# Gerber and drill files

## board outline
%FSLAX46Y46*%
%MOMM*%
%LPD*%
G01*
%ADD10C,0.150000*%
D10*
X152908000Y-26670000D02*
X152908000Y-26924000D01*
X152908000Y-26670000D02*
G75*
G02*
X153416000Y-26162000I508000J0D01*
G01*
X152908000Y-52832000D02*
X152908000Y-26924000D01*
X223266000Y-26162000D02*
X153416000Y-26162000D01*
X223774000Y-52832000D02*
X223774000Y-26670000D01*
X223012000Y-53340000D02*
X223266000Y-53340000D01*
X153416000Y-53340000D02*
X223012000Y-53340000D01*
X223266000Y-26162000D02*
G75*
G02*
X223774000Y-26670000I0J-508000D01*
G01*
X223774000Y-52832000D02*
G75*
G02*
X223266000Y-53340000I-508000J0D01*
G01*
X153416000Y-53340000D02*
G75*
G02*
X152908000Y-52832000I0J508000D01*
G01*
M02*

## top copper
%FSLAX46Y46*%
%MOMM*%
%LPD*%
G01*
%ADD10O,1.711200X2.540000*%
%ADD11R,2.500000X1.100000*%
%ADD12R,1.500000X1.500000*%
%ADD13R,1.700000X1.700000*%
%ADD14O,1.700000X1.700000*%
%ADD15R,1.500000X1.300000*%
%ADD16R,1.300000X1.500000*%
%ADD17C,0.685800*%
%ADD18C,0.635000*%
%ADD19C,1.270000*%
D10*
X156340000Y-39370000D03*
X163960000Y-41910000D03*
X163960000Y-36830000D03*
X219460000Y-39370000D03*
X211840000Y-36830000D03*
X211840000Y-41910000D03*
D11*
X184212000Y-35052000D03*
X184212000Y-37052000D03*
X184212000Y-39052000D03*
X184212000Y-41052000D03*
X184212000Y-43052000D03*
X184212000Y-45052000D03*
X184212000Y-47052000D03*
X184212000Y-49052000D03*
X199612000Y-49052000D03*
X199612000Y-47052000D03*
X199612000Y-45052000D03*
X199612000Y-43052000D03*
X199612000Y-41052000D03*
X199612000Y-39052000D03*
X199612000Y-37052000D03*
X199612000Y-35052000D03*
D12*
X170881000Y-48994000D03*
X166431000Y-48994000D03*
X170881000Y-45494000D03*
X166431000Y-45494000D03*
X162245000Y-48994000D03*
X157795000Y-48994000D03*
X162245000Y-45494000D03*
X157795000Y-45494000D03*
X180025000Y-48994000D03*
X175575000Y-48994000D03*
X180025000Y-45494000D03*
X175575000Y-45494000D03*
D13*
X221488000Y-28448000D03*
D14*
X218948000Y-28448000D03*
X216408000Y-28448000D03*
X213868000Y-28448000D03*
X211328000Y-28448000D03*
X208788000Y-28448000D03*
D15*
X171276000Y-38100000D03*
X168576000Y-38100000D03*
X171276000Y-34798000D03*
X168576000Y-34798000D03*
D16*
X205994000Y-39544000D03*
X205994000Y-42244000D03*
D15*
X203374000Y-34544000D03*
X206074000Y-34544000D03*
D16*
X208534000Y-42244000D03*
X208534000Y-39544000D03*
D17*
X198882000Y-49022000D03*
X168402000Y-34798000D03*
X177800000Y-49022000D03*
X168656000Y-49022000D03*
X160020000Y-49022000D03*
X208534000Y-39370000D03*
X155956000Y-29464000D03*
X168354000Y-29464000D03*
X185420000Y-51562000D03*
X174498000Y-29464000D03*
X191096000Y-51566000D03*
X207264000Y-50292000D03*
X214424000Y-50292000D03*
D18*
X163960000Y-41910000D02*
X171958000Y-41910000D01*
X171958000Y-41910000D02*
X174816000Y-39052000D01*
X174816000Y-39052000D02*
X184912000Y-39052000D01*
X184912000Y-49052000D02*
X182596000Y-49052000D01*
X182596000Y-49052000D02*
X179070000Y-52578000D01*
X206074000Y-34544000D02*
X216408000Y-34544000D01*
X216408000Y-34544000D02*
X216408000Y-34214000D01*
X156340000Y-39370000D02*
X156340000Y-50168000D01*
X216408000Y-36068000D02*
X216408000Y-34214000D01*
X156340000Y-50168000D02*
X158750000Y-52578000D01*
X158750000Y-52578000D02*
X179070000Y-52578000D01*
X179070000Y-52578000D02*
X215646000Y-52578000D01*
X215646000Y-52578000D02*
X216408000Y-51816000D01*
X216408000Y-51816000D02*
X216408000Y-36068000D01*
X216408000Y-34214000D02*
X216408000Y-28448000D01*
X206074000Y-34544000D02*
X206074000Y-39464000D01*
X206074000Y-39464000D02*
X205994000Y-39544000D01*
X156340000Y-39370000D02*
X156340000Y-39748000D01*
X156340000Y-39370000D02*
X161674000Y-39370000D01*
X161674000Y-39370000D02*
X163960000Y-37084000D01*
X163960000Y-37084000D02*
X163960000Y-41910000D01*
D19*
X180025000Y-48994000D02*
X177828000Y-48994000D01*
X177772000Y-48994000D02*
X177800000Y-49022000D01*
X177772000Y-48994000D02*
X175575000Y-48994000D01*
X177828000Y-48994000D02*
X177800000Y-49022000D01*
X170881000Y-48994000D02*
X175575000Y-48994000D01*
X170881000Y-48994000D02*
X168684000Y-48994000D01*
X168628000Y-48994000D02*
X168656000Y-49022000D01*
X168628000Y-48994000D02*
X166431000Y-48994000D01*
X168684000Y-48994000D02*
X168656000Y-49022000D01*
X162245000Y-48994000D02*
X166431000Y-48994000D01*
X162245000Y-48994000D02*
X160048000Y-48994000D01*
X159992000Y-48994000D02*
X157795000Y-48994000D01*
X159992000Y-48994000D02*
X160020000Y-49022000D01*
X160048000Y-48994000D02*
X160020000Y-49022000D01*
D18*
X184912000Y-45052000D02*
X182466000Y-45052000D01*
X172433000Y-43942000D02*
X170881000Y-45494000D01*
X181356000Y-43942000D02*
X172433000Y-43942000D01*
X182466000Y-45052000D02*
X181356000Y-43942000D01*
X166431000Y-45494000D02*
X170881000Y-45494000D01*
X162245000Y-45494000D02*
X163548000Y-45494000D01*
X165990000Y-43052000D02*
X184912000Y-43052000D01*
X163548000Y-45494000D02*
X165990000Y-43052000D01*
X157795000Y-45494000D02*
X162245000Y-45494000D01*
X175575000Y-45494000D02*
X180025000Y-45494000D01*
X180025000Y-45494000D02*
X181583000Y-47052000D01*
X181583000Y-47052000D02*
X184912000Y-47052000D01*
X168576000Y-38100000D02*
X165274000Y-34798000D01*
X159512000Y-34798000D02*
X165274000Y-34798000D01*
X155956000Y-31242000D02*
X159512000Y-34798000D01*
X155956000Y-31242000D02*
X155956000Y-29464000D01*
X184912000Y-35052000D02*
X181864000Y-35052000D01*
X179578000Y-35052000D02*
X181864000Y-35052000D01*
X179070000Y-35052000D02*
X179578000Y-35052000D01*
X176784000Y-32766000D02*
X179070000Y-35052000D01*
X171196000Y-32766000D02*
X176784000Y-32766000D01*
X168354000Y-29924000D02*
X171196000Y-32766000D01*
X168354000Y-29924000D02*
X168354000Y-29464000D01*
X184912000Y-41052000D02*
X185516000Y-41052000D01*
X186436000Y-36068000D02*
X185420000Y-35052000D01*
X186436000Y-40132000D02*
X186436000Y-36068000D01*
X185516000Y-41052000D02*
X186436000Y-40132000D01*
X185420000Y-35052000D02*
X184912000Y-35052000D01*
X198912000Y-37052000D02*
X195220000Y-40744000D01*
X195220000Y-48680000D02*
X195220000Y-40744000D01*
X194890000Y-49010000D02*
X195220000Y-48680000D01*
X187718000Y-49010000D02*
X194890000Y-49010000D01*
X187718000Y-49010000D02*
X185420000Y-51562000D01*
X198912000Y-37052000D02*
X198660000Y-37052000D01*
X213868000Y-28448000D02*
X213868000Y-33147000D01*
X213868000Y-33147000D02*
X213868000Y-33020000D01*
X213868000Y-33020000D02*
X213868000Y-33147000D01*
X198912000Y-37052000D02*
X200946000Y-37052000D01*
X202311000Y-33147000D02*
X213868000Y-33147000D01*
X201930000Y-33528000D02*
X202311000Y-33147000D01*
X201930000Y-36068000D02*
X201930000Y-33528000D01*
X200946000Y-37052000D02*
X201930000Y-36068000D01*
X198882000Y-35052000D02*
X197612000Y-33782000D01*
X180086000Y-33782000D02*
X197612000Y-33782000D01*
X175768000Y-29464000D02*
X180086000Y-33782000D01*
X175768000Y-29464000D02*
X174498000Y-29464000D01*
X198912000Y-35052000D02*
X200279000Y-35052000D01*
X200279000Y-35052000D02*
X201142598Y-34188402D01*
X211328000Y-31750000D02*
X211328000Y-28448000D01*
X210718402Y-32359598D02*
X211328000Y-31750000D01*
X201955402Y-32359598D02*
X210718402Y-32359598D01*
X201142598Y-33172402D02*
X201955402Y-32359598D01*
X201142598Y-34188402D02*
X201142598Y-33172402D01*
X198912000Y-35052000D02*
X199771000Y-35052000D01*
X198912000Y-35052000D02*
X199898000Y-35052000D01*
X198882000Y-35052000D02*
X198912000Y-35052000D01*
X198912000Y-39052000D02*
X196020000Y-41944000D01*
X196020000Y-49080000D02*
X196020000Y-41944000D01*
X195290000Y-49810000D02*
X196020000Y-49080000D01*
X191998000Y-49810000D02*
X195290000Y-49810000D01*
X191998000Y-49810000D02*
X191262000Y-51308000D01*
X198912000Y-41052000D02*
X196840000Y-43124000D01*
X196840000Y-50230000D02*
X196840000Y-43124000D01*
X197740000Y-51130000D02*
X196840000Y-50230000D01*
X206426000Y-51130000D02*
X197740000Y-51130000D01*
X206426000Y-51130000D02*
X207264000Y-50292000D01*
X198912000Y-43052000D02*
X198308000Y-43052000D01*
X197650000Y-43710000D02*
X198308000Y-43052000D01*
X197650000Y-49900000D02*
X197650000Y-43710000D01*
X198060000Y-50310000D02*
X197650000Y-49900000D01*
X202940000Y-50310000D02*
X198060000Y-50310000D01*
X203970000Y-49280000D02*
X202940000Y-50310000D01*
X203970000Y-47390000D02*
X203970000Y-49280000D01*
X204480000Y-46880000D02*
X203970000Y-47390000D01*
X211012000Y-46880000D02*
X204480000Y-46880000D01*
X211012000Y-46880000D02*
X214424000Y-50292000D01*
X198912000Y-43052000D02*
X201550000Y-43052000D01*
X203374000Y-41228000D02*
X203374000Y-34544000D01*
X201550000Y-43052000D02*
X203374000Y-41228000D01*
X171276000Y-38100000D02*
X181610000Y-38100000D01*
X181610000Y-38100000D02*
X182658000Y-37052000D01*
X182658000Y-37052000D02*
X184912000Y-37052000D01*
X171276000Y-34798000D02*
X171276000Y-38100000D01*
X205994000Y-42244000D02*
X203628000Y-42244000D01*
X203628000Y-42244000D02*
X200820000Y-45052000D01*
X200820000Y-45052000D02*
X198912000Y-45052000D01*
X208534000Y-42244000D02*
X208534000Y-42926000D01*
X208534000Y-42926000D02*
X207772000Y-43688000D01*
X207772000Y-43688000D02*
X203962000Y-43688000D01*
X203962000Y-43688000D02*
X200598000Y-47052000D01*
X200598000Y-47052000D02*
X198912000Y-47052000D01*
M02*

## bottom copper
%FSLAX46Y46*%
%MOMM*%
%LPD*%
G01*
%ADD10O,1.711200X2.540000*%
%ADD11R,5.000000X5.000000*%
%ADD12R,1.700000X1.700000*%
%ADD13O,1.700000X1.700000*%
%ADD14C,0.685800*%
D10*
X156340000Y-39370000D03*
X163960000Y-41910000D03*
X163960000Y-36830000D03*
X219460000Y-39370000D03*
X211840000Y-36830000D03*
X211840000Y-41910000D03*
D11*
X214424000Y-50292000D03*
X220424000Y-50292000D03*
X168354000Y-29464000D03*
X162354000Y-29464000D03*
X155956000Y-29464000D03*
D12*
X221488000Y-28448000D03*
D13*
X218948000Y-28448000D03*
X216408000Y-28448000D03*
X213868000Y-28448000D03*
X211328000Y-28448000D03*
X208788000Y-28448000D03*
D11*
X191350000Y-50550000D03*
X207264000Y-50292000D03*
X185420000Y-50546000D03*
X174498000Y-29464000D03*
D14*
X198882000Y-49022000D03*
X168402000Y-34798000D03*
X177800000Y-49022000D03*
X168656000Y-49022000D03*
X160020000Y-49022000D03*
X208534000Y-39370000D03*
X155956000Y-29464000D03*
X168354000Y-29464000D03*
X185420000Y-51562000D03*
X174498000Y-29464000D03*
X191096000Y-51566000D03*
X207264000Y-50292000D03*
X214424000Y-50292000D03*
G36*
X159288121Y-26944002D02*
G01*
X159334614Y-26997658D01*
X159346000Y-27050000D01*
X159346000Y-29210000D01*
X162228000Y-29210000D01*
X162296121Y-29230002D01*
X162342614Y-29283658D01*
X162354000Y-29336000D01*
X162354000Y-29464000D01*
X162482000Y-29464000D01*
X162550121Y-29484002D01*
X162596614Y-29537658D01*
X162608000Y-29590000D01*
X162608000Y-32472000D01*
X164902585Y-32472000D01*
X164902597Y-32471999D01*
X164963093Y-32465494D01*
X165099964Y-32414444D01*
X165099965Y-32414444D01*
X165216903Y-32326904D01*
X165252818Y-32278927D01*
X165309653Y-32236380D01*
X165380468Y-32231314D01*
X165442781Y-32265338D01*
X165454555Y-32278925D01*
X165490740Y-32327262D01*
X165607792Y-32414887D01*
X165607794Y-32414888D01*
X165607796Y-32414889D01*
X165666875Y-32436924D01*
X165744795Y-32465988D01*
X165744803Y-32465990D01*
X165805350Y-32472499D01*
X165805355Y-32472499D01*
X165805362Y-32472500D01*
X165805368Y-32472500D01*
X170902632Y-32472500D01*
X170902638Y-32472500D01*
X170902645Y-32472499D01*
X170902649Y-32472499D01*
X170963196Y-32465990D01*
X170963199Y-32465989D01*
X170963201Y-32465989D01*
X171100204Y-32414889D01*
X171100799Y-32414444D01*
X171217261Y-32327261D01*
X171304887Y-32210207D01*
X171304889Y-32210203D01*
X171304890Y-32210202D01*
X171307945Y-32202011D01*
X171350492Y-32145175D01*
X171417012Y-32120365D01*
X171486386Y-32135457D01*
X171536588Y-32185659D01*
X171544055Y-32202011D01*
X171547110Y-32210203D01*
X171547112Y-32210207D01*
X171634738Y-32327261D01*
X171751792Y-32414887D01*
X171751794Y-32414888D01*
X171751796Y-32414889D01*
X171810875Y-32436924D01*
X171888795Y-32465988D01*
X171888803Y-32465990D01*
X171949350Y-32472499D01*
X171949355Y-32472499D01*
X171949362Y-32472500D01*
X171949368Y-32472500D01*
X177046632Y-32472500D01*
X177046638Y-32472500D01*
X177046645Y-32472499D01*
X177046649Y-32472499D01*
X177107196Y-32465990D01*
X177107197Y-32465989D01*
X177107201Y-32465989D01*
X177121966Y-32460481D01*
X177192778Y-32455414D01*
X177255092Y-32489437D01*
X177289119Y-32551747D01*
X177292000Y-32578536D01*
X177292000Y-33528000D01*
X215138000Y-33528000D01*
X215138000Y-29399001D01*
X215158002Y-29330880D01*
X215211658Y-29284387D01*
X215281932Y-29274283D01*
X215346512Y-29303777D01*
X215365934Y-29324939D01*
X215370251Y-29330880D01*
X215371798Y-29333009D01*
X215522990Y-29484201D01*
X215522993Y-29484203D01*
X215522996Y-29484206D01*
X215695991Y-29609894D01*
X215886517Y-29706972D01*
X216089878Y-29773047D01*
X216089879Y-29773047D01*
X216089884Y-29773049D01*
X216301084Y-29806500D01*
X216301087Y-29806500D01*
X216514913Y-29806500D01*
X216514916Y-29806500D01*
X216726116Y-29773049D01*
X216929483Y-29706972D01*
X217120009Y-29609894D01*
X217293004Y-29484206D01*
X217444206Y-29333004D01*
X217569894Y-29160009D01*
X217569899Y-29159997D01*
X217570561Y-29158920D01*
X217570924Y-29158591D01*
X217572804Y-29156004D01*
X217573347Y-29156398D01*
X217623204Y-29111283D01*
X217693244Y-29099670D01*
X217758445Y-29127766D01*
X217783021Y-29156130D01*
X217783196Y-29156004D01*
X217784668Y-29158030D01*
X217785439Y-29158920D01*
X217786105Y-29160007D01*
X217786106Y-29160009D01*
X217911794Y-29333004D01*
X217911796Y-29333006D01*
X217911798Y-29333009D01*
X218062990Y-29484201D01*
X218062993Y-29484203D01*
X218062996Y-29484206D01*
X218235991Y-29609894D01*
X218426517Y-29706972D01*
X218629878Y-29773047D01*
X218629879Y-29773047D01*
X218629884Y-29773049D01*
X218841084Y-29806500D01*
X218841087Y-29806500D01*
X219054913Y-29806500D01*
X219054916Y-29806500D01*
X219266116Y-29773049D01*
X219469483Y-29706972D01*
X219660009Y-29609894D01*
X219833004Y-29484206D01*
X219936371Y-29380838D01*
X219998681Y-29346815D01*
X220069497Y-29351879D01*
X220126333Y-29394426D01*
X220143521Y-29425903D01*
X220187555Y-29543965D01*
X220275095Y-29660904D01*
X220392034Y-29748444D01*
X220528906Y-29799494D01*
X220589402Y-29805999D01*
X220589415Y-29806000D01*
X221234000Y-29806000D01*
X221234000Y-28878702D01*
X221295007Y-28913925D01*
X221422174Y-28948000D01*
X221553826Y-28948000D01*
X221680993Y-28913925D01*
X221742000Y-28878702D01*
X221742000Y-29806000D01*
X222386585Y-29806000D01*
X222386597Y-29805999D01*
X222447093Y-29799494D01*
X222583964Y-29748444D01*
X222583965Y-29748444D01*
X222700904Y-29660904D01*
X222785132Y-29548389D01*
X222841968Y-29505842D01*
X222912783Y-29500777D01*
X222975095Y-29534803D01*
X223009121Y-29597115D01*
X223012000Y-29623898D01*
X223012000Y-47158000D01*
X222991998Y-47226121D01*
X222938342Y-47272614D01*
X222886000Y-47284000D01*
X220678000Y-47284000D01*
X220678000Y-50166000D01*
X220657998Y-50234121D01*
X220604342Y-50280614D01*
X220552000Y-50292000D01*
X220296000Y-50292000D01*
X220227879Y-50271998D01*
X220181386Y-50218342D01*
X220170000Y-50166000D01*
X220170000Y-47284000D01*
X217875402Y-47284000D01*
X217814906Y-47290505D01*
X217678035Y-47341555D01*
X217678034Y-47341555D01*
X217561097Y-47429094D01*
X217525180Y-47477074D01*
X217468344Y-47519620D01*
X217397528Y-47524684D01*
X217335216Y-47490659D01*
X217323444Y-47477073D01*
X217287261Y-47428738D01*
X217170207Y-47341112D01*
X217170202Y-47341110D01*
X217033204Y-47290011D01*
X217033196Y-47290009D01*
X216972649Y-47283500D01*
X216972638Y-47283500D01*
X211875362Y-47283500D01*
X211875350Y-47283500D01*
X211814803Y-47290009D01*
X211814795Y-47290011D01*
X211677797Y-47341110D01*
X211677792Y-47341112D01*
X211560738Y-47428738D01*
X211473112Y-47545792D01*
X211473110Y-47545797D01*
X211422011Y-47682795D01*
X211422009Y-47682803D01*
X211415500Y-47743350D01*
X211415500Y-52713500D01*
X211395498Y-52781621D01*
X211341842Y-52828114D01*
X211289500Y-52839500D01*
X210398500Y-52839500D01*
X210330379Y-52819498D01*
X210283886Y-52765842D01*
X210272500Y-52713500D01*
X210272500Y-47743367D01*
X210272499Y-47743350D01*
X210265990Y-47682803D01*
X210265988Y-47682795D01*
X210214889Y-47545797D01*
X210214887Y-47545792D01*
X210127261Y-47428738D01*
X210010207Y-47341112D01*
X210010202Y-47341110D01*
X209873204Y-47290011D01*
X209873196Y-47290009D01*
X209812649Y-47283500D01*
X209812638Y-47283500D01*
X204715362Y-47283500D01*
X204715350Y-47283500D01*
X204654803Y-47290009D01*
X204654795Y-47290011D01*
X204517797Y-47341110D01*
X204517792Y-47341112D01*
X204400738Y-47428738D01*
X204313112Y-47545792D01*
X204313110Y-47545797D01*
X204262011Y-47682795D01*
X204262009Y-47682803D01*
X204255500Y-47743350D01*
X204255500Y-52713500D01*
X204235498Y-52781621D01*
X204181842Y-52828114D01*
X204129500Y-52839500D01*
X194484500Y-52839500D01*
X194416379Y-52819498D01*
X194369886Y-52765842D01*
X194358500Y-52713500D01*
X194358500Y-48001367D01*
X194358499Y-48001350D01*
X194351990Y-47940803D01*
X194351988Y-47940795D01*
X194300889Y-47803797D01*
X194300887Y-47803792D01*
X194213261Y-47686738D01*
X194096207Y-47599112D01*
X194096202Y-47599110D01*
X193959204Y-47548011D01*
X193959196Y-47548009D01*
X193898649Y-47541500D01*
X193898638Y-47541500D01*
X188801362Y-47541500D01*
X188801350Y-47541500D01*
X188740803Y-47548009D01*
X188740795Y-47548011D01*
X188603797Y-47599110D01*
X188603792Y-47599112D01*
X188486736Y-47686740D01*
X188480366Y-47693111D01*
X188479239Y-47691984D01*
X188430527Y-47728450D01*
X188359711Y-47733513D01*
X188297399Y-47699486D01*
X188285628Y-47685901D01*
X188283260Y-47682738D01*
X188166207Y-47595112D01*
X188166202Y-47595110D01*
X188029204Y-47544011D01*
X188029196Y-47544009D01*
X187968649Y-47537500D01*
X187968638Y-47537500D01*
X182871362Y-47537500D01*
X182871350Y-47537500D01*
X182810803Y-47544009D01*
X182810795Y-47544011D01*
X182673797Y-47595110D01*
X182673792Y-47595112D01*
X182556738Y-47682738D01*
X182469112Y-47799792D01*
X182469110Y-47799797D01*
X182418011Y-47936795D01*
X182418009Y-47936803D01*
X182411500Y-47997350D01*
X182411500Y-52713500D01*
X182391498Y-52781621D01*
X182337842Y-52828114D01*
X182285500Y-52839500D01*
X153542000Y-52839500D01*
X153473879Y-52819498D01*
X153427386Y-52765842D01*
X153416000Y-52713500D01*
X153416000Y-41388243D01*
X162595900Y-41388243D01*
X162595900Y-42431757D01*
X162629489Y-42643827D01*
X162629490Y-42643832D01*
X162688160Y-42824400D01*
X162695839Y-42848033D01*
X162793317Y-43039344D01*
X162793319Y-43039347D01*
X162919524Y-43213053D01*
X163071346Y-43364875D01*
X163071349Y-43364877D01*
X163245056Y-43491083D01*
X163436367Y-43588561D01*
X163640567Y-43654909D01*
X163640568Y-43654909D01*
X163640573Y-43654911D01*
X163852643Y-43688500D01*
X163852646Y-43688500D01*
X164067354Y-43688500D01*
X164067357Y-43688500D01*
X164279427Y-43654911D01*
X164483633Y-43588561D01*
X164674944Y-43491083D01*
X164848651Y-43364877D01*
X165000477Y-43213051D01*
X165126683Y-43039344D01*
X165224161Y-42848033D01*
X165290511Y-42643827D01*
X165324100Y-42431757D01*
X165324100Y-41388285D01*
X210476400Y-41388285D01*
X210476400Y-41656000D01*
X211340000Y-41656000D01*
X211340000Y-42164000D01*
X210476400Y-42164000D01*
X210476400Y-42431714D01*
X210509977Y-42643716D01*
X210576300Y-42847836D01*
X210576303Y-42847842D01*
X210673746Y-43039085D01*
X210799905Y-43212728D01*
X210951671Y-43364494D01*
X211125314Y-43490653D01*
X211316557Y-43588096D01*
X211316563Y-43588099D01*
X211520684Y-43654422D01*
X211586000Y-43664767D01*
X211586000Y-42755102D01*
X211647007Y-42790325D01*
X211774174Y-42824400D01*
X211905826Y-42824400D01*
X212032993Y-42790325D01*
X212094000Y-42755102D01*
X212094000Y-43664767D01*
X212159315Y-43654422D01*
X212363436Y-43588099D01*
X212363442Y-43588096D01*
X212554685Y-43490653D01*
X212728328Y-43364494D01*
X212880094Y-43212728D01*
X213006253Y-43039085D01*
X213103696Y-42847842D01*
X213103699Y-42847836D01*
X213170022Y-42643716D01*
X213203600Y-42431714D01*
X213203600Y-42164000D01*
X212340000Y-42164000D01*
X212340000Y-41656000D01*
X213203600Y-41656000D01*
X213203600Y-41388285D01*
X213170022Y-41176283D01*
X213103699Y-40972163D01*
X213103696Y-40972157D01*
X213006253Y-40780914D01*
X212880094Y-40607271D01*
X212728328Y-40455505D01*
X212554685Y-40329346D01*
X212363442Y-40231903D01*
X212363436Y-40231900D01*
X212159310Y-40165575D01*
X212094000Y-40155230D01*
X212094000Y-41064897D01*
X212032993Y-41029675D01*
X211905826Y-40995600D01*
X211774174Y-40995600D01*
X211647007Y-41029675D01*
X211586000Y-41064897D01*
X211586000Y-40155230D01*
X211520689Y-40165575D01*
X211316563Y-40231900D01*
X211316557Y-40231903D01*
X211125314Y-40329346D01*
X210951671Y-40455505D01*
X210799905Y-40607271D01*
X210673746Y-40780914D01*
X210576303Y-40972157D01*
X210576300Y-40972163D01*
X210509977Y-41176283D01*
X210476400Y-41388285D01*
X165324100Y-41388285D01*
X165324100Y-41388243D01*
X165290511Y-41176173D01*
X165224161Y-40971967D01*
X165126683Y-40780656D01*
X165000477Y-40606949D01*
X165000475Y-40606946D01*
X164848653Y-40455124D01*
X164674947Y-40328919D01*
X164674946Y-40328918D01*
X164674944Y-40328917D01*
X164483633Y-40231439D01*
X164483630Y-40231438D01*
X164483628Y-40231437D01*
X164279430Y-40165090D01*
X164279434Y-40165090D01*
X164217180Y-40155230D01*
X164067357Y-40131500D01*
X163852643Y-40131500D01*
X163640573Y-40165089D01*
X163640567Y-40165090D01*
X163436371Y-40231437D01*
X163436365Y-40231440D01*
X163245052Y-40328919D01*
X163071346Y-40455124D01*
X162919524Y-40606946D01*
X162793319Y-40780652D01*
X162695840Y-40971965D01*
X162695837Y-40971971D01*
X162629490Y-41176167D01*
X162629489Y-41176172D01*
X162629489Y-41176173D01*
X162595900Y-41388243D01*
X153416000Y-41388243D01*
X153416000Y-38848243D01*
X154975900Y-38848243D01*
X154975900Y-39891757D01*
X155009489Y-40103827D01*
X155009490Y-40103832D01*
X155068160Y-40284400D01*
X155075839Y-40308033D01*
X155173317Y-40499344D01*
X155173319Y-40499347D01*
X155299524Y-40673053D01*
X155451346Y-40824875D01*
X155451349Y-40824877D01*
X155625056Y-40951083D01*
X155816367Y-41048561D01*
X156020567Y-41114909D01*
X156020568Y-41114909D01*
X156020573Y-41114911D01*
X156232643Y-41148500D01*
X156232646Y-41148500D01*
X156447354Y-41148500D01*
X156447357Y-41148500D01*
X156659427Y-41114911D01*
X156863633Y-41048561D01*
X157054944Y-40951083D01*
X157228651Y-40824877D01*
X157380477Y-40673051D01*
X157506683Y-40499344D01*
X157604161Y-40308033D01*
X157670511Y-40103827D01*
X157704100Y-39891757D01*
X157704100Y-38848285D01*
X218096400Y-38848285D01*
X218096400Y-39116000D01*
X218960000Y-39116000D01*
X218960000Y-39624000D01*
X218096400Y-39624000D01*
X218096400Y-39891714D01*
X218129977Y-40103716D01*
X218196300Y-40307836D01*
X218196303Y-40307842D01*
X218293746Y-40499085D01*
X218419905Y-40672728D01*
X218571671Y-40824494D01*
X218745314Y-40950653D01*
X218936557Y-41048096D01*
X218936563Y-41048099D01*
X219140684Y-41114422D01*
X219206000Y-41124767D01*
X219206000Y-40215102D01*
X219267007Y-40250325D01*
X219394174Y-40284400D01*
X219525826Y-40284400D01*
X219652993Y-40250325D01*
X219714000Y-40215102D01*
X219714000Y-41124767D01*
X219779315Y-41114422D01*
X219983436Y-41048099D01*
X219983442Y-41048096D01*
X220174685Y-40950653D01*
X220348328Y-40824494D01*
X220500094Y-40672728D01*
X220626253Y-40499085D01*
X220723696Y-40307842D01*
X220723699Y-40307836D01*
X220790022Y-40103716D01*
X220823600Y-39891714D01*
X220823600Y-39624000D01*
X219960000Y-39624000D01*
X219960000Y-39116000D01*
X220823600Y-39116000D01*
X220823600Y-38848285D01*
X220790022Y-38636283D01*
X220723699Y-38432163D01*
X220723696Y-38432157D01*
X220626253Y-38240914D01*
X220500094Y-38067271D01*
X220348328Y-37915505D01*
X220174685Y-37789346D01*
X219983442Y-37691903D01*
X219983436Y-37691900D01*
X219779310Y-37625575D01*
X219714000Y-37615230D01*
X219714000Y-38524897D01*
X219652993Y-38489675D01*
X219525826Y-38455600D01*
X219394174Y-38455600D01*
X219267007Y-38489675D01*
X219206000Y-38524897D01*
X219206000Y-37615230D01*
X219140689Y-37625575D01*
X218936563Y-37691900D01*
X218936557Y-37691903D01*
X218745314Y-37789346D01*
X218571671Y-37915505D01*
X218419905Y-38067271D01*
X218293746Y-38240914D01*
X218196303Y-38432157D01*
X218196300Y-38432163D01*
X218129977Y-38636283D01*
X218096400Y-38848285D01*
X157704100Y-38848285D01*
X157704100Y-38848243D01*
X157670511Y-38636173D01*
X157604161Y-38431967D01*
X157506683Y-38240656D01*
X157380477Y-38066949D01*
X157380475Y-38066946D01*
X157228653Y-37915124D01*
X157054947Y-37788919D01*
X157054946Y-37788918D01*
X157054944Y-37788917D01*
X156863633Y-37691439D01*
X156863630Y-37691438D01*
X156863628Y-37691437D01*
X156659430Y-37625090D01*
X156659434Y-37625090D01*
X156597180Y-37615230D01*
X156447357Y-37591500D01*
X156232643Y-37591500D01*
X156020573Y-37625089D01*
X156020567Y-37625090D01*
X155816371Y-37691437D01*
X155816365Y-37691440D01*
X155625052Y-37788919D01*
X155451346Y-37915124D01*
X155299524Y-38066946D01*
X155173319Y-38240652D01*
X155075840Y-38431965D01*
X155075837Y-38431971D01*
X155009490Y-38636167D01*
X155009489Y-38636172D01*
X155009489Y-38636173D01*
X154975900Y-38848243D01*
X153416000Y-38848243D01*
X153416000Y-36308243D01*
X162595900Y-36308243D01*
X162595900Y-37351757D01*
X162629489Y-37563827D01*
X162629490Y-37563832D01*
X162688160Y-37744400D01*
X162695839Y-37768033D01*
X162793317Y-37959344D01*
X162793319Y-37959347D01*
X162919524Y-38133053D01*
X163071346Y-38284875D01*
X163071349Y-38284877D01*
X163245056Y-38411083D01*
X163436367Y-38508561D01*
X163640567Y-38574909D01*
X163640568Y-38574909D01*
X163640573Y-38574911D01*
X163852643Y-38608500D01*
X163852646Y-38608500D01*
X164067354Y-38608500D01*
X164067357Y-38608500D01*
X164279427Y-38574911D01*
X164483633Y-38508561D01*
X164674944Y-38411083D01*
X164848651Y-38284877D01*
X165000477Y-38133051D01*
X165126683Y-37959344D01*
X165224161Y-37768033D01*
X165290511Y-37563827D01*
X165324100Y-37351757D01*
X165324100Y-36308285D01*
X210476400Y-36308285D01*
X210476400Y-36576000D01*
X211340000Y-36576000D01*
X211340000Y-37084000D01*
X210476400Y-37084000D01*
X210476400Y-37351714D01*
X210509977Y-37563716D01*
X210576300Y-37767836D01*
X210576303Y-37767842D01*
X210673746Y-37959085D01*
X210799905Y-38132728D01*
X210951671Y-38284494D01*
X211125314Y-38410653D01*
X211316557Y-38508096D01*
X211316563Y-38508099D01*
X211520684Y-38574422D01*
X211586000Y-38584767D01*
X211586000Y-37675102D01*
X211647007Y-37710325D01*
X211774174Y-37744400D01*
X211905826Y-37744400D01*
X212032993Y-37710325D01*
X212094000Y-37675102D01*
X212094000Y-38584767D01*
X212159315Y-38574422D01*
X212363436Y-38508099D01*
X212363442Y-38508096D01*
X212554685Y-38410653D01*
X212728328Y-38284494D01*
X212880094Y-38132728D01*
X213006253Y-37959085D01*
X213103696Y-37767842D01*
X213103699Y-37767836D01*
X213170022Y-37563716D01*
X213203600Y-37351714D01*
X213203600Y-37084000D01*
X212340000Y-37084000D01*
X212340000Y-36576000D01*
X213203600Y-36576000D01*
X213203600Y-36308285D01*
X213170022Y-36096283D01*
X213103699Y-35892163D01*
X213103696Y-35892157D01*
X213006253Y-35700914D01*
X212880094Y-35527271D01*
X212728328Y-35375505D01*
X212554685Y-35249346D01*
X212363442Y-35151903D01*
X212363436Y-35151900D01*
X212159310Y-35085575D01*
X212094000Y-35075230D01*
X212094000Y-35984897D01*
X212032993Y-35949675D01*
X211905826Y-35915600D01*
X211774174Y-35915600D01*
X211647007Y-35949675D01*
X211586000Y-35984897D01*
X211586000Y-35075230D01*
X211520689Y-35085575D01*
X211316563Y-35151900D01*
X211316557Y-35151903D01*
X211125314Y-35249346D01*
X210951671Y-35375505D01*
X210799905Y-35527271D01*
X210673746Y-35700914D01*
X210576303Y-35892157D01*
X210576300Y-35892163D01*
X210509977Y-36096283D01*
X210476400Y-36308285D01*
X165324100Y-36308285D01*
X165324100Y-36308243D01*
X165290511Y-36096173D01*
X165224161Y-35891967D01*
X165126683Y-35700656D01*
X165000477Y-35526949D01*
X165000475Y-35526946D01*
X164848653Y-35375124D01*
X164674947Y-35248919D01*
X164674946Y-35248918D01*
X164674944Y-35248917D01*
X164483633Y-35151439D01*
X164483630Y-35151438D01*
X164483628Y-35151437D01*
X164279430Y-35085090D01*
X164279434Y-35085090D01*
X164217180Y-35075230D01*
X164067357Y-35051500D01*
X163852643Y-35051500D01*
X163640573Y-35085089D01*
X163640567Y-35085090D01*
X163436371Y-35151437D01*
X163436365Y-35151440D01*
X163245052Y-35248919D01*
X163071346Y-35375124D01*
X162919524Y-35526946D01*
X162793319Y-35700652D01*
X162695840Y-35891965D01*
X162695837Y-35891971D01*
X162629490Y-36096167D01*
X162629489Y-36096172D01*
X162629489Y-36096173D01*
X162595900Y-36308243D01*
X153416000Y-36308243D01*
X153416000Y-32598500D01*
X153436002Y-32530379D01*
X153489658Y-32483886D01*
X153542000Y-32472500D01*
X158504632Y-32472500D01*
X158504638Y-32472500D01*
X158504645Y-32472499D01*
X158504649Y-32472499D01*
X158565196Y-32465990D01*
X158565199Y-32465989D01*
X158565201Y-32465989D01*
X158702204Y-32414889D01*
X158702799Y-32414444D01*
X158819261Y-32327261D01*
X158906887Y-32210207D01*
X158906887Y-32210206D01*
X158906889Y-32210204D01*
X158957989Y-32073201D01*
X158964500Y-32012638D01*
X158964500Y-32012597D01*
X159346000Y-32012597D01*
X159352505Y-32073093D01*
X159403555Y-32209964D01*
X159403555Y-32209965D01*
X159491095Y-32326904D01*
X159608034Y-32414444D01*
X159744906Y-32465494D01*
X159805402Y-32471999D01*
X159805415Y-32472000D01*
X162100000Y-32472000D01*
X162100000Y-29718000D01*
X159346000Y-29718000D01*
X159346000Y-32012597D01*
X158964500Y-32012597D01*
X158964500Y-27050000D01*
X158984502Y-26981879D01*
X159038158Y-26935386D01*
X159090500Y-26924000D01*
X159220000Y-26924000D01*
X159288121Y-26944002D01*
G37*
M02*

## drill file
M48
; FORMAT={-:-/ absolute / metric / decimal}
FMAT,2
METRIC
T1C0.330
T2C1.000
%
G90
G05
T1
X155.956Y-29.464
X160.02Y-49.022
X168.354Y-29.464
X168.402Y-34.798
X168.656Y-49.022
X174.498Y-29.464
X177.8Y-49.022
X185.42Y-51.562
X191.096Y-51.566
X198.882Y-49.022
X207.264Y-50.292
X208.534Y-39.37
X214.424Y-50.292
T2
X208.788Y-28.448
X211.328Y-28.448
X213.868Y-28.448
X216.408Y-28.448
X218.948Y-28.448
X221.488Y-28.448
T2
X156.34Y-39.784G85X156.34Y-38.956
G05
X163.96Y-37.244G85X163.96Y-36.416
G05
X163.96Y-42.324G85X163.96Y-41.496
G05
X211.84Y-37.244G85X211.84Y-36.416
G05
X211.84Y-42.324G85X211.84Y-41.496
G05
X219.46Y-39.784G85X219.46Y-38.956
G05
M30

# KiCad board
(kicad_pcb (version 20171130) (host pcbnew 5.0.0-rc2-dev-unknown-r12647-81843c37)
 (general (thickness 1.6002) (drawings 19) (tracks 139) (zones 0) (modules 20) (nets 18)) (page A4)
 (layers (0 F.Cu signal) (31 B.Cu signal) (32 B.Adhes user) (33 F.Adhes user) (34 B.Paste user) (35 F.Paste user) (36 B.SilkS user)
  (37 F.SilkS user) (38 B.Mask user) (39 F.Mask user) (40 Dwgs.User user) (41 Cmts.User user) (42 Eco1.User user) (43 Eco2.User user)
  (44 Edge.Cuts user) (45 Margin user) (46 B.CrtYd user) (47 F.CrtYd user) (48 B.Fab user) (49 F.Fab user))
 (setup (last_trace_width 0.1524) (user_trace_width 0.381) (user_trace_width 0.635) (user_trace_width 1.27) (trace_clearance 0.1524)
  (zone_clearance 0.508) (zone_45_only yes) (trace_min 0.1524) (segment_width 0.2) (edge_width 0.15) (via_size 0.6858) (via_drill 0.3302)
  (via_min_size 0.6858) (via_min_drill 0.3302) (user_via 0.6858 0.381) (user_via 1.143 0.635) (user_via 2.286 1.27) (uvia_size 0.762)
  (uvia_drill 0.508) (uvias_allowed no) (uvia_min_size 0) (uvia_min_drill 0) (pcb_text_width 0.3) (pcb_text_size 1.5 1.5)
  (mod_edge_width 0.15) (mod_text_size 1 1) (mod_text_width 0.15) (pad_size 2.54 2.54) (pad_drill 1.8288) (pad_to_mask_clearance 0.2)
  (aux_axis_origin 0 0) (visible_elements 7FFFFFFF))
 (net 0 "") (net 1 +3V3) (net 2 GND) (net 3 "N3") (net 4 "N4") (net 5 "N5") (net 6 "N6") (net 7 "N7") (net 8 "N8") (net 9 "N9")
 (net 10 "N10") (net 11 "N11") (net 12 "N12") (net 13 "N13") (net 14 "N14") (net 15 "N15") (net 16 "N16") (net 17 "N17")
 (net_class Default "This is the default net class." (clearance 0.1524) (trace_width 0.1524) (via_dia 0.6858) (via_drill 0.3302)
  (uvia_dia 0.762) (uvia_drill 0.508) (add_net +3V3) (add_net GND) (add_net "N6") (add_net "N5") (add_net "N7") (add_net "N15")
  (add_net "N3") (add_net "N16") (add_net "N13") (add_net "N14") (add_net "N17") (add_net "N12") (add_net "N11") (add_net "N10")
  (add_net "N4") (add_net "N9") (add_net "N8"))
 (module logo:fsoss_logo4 (layer F.Cu) (at 208.788 45.085)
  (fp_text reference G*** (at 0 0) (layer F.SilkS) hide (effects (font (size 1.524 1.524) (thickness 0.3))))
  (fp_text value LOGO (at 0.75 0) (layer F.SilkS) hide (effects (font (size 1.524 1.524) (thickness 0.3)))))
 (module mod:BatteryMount (layer F.Cu) (at 187.96 39.37 90)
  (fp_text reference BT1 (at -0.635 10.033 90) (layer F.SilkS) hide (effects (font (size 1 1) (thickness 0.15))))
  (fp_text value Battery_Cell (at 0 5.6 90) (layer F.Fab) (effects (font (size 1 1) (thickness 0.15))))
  (pad 1 thru_hole oval (at 0 -31.62 90) (size 2.54 1.7112) (drill oval 1.8288 1) (layers *.Cu *.Mask) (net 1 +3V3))
  (pad 1 thru_hole oval (at -2.54 -24 90) (size 2.54 1.7112) (drill oval 1.8288 1) (layers *.Cu *.Mask) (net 1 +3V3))
  (pad 1 thru_hole oval (at 2.54 -24 90) (size 2.54 1.7112) (drill oval 1.8288 1) (layers *.Cu *.Mask) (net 1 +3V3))
  (pad 2 thru_hole oval (at 0 31.5 90) (size 2.54 1.7112) (drill oval 1.8288 1) (layers *.Cu *.Mask) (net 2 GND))
  (pad 2 thru_hole oval (at 2.54 23.88 90) (size 2.54 1.7112) (drill oval 1.8288 1) (layers *.Cu *.Mask) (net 2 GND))
  (pad 2 thru_hole oval (at -2.54 23.88 90) (size 2.54 1.7112) (drill oval 1.8288 1) (layers *.Cu *.Mask) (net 2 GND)))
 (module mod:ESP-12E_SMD (layer F.Cu) (at 184.912 35.052)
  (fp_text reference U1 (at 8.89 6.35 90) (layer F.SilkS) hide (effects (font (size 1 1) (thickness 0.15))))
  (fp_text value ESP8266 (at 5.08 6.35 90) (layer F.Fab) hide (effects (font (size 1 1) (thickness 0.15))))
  (pad 1 smd rect (at 0 0) (size 2.5 1.1) (drill (offset -0.7 0)) (layers F.Cu F.Paste F.Mask) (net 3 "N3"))
  (pad 2 smd rect (at 0 2) (size 2.5 1.1) (drill (offset -0.7 0)) (layers F.Cu F.Paste F.Mask) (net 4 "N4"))
  (pad 3 smd rect (at 0 4) (size 2.5 1.1) (drill (offset -0.7 0)) (layers F.Cu F.Paste F.Mask) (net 1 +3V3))
  (pad 4 smd rect (at 0 6) (size 2.5 1.1) (drill (offset -0.7 0)) (layers F.Cu F.Paste F.Mask) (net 3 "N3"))
  (pad 5 smd rect (at 0 8) (size 2.5 1.1) (drill (offset -0.7 0)) (layers F.Cu F.Paste F.Mask) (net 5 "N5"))
  (pad 6 smd rect (at 0 10) (size 2.5 1.1) (drill (offset -0.7 0)) (layers F.Cu F.Paste F.Mask) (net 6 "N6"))
  (pad 7 smd rect (at 0 12) (size 2.5 1.1) (drill (offset -0.7 0)) (layers F.Cu F.Paste F.Mask) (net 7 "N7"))
  (pad 8 smd rect (at 0 14) (size 2.5 1.1) (drill (offset -0.7 0)) (layers F.Cu F.Paste F.Mask) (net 1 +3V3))
  (pad 9 smd rect (at 14 14) (size 2.5 1.1) (drill (offset 0.7 0)) (layers F.Cu F.Paste F.Mask) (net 2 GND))
  (pad 10 smd rect (at 14 12) (size 2.5 1.1) (drill (offset 0.7 0)) (layers F.Cu F.Paste F.Mask) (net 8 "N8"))
  (pad 11 smd rect (at 14 10) (size 2.5 1.1) (drill (offset 0.7 0)) (layers F.Cu F.Paste F.Mask) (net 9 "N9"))
  (pad 12 smd rect (at 14 8) (size 2.5 1.1) (drill (offset 0.7 0)) (layers F.Cu F.Paste F.Mask) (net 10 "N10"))
  (pad 13 smd rect (at 14 6) (size 2.5 1.1) (drill (offset 0.7 0)) (layers F.Cu F.Paste F.Mask) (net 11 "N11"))
  (pad 14 smd rect (at 14 4) (size 2.5 1.1) (drill (offset 0.7 0)) (layers F.Cu F.Paste F.Mask) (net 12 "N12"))
  (pad 15 smd rect (at 14 2) (size 2.5 1.1) (drill (offset 0.7 0)) (layers F.Cu F.Paste F.Mask) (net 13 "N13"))
  (pad 16 smd rect (at 14 0) (size 2.5 1.1) (drill (offset 0.7 0)) (layers F.Cu F.Paste F.Mask) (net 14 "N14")))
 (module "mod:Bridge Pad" (layer F.Cu) (at 217.424 50.292 180)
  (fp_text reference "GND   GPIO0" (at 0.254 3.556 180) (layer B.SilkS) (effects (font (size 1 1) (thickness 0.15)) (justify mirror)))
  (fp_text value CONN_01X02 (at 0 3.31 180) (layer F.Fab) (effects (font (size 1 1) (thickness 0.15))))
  (pad 1 smd rect (at 3 0 180) (size 5 5) (layers B.Cu B.Mask) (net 10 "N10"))
  (pad 2 smd rect (at -3 0 180) (size 5 5) (layers B.Cu B.Mask) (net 2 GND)))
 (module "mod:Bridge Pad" (layer F.Cu) (at 165.354 29.464)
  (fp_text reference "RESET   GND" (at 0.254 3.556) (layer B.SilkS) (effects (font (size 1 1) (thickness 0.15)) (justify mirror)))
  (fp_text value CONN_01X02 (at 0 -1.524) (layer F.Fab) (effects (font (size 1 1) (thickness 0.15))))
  (pad 1 smd rect (at 3 0) (size 5 5) (layers B.Cu B.Mask) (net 3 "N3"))
  (pad 2 smd rect (at -3 0) (size 5 5) (layers B.Cu B.Mask) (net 2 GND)))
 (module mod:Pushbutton (layer F.Cu) (at 168.656 47.244 180)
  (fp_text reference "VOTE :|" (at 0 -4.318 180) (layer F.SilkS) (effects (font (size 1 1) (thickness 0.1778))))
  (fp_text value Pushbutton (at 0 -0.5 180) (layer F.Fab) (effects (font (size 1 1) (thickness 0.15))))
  (pad 1 smd rect (at -2.225 -1.75 180) (size 1.5 1.5) (layers F.Cu F.Paste F.Mask) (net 2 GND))
  (pad 1 smd rect (at 2.225 -1.75 180) (size 1.5 1.5) (layers F.Cu F.Paste F.Mask) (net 2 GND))
  (pad 2 smd rect (at -2.225 1.75 180) (size 1.5 1.5) (layers F.Cu F.Paste F.Mask) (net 6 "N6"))
  (pad 2 smd rect (at 2.225 1.75 180) (size 1.5 1.5) (layers F.Cu F.Paste F.Mask) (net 6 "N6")))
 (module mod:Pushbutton (layer F.Cu) (at 160.02 47.244 180)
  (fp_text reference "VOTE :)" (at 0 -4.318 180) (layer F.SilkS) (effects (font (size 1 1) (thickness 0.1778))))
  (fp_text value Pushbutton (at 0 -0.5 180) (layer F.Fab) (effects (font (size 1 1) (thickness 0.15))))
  (pad 1 smd rect (at -2.225 -1.75 180) (size 1.5 1.5) (layers F.Cu F.Paste F.Mask) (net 2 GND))
  (pad 1 smd rect (at 2.225 -1.75 180) (size 1.5 1.5) (layers F.Cu F.Paste F.Mask) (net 2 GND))
  (pad 2 smd rect (at -2.225 1.75 180) (size 1.5 1.5) (layers F.Cu F.Paste F.Mask) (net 5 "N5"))
  (pad 2 smd rect (at 2.225 1.75 180) (size 1.5 1.5) (layers F.Cu F.Paste F.Mask) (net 5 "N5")))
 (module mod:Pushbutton (layer F.Cu) (at 177.8 47.244 180)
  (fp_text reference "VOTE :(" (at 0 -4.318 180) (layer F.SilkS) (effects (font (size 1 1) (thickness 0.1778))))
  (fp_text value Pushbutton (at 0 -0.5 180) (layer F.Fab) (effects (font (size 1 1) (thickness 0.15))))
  (pad 1 smd rect (at -2.225 -1.75 180) (size 1.5 1.5) (layers F.Cu F.Paste F.Mask) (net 2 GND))
  (pad 1 smd rect (at 2.225 -1.75 180) (size 1.5 1.5) (layers F.Cu F.Paste F.Mask) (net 2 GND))
  (pad 2 smd rect (at -2.225 1.75 180) (size 1.5 1.5) (layers F.Cu F.Paste F.Mask) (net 7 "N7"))
  (pad 2 smd rect (at 2.225 1.75 180) (size 1.5 1.5) (layers F.Cu F.Paste F.Mask) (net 7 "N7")))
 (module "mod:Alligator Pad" (layer F.Cu) (at 155.956 29.464)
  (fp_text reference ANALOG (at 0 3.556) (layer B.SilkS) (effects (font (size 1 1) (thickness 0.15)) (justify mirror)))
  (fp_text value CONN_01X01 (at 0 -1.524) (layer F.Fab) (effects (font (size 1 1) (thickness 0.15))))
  (pad 1 smd rect (at 0 0) (size 5 5) (layers B.Cu B.Mask) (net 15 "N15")))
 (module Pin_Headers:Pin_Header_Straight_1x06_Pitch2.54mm (layer B.Cu) (at 221.488 28.448 90)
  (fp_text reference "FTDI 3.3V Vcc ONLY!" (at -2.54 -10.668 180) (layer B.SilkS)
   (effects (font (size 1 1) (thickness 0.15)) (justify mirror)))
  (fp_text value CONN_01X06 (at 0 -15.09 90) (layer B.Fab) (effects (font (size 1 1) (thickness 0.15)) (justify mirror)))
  (pad 1 thru_hole rect (at 0 0 90) (size 1.7 1.7) (drill 1) (layers *.Cu *.Mask) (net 2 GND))
  (pad 2 thru_hole oval (at 0 -2.54 90) (size 1.7 1.7) (drill 1) (layers *.Cu *.Mask) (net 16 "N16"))
  (pad 3 thru_hole oval (at 0 -5.08 90) (size 1.7 1.7) (drill 1) (layers *.Cu *.Mask) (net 1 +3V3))
  (pad 4 thru_hole oval (at 0 -7.62 90) (size 1.7 1.7) (drill 1) (layers *.Cu *.Mask) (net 13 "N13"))
  (pad 5 thru_hole oval (at 0 -10.16 90) (size 1.7 1.7) (drill 1) (layers *.Cu *.Mask) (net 14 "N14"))
  (pad 6 thru_hole oval (at 0 -12.7 90) (size 1.7 1.7) (drill 1) (layers *.Cu *.Mask) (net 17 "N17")))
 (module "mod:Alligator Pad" (layer F.Cu) (at 191.35 50.55)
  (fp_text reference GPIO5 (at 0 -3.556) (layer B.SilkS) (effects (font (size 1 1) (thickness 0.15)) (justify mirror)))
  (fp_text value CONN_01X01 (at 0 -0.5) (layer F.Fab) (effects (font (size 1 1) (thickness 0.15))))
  (pad 1 smd rect (at 0 0) (size 5 5) (layers B.Cu B.Mask) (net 12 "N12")))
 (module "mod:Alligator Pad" (layer F.Cu) (at 207.264 50.292)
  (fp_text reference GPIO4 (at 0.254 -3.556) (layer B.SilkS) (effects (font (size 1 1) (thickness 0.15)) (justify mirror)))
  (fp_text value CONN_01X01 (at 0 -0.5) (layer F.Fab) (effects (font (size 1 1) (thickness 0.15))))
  (pad 1 smd rect (at 0 0) (size 5 5) (layers B.Cu B.Mask) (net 11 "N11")))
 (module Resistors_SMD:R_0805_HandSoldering (layer F.Cu) (at 169.926 38.1 180)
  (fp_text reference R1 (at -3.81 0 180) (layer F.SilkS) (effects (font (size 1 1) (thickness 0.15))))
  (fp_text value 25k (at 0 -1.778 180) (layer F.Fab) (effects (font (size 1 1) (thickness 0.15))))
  (pad 1 smd rect (at -1.35 0 180) (size 1.5 1.3) (layers F.Cu F.Paste F.Mask) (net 4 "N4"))
  (pad 2 smd rect (at 1.35 0 180) (size 1.5 1.3) (layers F.Cu F.Paste F.Mask) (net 15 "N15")))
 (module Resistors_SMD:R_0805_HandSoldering (layer F.Cu) (at 169.926 34.798 180)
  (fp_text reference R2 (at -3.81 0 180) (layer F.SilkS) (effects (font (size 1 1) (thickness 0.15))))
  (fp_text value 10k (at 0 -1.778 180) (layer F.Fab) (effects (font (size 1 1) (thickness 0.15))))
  (pad 1 smd rect (at -1.35 0 180) (size 1.5 1.3) (layers F.Cu F.Paste F.Mask) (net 4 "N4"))
  (pad 2 smd rect (at 1.35 0 180) (size 1.5 1.3) (layers F.Cu F.Paste F.Mask) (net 2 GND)))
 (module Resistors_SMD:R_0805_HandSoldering (layer F.Cu) (at 205.994 40.894 270)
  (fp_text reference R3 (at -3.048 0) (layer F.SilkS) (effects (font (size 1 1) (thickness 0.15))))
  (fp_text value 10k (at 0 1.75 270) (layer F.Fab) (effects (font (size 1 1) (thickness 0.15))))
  (pad 1 smd rect (at -1.35 0 270) (size 1.5 1.3) (layers F.Cu F.Paste F.Mask) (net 1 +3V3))
  (pad 2 smd rect (at 1.35 0 270) (size 1.5 1.3) (layers F.Cu F.Paste F.Mask) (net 9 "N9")))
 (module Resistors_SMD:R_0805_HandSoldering (layer F.Cu) (at 204.724 34.544)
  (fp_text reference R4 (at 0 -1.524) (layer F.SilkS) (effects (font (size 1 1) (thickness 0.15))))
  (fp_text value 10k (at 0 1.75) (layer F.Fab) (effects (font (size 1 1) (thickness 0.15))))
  (pad 1 smd rect (at -1.35 0) (size 1.5 1.3) (layers F.Cu F.Paste F.Mask) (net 10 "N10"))
  (pad 2 smd rect (at 1.35 0) (size 1.5 1.3) (layers F.Cu F.Paste F.Mask) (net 1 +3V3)))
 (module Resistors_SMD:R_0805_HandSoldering (layer F.Cu) (at 208.534 40.894 90)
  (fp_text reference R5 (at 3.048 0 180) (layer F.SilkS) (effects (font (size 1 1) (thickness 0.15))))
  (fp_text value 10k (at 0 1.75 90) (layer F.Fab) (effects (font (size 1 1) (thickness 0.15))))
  (pad 1 smd rect (at -1.35 0 90) (size 1.5 1.3) (layers F.Cu F.Paste F.Mask) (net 8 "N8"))
  (pad 2 smd rect (at 1.35 0 90) (size 1.5 1.3) (layers F.Cu F.Paste F.Mask) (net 2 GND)))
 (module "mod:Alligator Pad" (layer F.Cu) (at 185.42 50.546)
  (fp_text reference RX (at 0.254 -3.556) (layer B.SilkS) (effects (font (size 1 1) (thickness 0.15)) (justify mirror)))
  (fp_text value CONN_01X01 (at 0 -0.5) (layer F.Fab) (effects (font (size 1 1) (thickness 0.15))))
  (pad 1 smd rect (at 0 0) (size 5 5) (layers B.Cu B.Mask) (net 13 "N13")))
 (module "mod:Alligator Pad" (layer F.Cu) (at 174.498 29.464)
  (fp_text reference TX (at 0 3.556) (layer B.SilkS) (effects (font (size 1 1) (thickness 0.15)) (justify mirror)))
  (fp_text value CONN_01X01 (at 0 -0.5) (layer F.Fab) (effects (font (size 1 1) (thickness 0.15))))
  (pad 1 smd rect (at 0 0) (size 5 5) (layers B.Cu B.Mask) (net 14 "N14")))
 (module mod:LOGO (layer F.Cu) (at 159.258 31.242)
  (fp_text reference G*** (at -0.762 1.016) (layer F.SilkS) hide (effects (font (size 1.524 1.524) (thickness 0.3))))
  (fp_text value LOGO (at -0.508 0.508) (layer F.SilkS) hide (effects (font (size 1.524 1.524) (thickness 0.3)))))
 (gr_line (start 152.908 26.67) (end 152.908 26.924) (angle 90) (layer Edge.Cuts) (width 0.15))
 (gr_arc (start 153.416 26.67) (end 152.908 26.67) (angle 90) (layer Edge.Cuts) (width 0.15))
 (gr_line (start 152.908 52.832) (end 152.908 26.924) (angle 90) (layer Edge.Cuts) (width 0.15))
 (gr_line (start 223.266 26.162) (end 153.416 26.162) (angle 90) (layer Edge.Cuts) (width 0.15))
 (gr_line (start 223.774 52.832) (end 223.774 26.67) (angle 90) (layer Edge.Cuts) (width 0.15))
 (gr_line (start 223.012 53.34) (end 223.266 53.34) (angle 90) (layer Edge.Cuts) (width 0.15))
 (gr_line (start 153.416 53.34) (end 223.012 53.34) (angle 90) (layer Edge.Cuts) (width 0.15))
 (gr_arc (start 223.266 26.67) (end 223.266 26.162) (angle 90) (layer Edge.Cuts) (width 0.15))
 (gr_arc (start 223.266 52.832) (end 223.774 52.832) (angle 90) (layer Edge.Cuts) (width 0.15))
 (gr_arc (start 153.416 52.832) (end 153.416 53.34) (angle 90) (layer Edge.Cuts) (width 0.15))
 (segment (start 163.96 41.91) (end 171.958 41.91) (width 0.635) (layer F.Cu) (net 1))
 (segment (start 171.958 41.91) (end 174.816 39.052) (width 0.635) (layer F.Cu) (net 1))
 (segment (start 174.816 39.052) (end 184.912 39.052) (width 0.635) (layer F.Cu) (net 1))
 (segment (start 184.912 49.052) (end 182.596 49.052) (width 0.635) (layer F.Cu) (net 1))
 (segment (start 182.596 49.052) (end 179.07 52.578) (width 0.635) (layer F.Cu) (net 1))
 (segment (start 206.074 34.544) (end 216.408 34.544) (width 0.635) (layer F.Cu) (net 1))
 (segment (start 216.408 34.544) (end 216.408 34.214) (width 0.635) (layer F.Cu) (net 1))
 (segment (start 156.34 39.37) (end 156.34 50.168) (width 0.635) (layer F.Cu) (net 1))
 (segment (start 216.408 36.068) (end 216.408 34.214) (width 0.635) (layer F.Cu) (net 1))
 (segment (start 156.34 50.168) (end 158.75 52.578) (width 0.635) (layer F.Cu) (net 1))
 (segment (start 158.75 52.578) (end 179.07 52.578) (width 0.635) (layer F.Cu) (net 1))
 (segment (start 179.07 52.578) (end 215.646 52.578) (width 0.635) (layer F.Cu) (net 1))
 (segment (start 215.646 52.578) (end 216.408 51.816) (width 0.635) (layer F.Cu) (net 1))
 (segment (start 216.408 51.816) (end 216.408 36.068) (width 0.635) (layer F.Cu) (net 1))
 (segment (start 216.408 34.214) (end 216.408 28.448) (width 0.635) (layer F.Cu) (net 1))
 (segment (start 206.074 34.544) (end 206.074 39.464) (width 0.635) (layer F.Cu) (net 1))
 (segment (start 206.074 39.464) (end 205.994 39.544) (width 0.635) (layer F.Cu) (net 1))
 (segment (start 156.34 39.37) (end 156.34 39.748) (width 0.635) (layer F.Cu) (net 1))
 (segment (start 156.34 39.37) (end 161.674 39.37) (width 0.635) (layer F.Cu) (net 1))
 (segment (start 161.674 39.37) (end 163.96 37.084) (width 0.635) (layer F.Cu) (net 1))
 (segment (start 163.96 37.084) (end 163.96 41.91) (width 0.635) (layer F.Cu) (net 1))
 (via (at 198.882 49.022) (size 0.6858) (drill 0.3302) (layers F.Cu B.Cu) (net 2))
 (via (at 168.402 34.798) (size 0.6858) (drill 0.3302) (layers F.Cu B.Cu) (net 2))
 (segment (start 180.025 48.994) (end 177.828 48.994) (width 1.27) (layer F.Cu) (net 2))
 (segment (start 177.772 48.994) (end 177.8 49.022) (width 1.27) (layer F.Cu) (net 2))
 (via (at 177.8 49.022) (size 0.6858) (drill 0.3302) (layers F.Cu B.Cu) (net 2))
 (segment (start 177.772 48.994) (end 175.575 48.994) (width 1.27) (layer F.Cu) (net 2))
 (segment (start 177.828 48.994) (end 177.8 49.022) (width 1.27) (layer F.Cu) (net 2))
 (segment (start 170.881 48.994) (end 175.575 48.994) (width 1.27) (layer F.Cu) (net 2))
 (segment (start 170.881 48.994) (end 168.684 48.994) (width 1.27) (layer F.Cu) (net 2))
 (segment (start 168.628 48.994) (end 168.656 49.022) (width 1.27) (layer F.Cu) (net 2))
 (via (at 168.656 49.022) (size 0.6858) (drill 0.3302) (layers F.Cu B.Cu) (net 2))
 (segment (start 168.628 48.994) (end 166.431 48.994) (width 1.27) (layer F.Cu) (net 2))
 (segment (start 168.684 48.994) (end 168.656 49.022) (width 1.27) (layer F.Cu) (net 2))
 (segment (start 162.245 48.994) (end 166.431 48.994) (width 1.27) (layer F.Cu) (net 2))
 (segment (start 162.245 48.994) (end 160.048 48.994) (width 1.27) (layer F.Cu) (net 2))
 (segment (start 159.992 48.994) (end 157.795 48.994) (width 1.27) (layer F.Cu) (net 2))
 (via (at 160.02 49.022) (size 0.6858) (drill 0.3302) (layers F.Cu B.Cu) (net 2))
 (segment (start 159.992 48.994) (end 160.02 49.022) (width 1.27) (layer F.Cu) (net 2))
 (segment (start 160.048 48.994) (end 160.02 49.022) (width 1.27) (layer F.Cu) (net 2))
 (via (at 208.534 39.37) (size 0.6858) (drill 0.3302) (layers F.Cu B.Cu) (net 2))
 (segment (start 184.912 45.052) (end 182.466 45.052) (width 0.635) (layer F.Cu) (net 6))
 (segment (start 172.433 43.942) (end 170.881 45.494) (width 0.635) (layer F.Cu) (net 6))
 (segment (start 181.356 43.942) (end 172.433 43.942) (width 0.635) (layer F.Cu) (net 6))
 (segment (start 182.466 45.052) (end 181.356 43.942) (width 0.635) (layer F.Cu) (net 6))
 (segment (start 166.431 45.494) (end 170.881 45.494) (width 0.635) (layer F.Cu) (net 6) (status 30))
 (segment (start 162.245 45.494) (end 163.548 45.494) (width 0.635) (layer F.Cu) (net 5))
 (segment (start 165.99 43.052) (end 184.912 43.052) (width 0.635) (layer F.Cu) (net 5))
 (segment (start 163.548 45.494) (end 165.99 43.052) (width 0.635) (layer F.Cu) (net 5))
 (segment (start 157.795 45.494) (end 162.245 45.494) (width 0.635) (layer F.Cu) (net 5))
 (segment (start 175.575 45.494) (end 180.025 45.494) (width 0.635) (layer F.Cu) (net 7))
 (segment (start 180.025 45.494) (end 181.583 47.052) (width 0.635) (layer F.Cu) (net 7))
 (segment (start 181.583 47.052) (end 184.912 47.052) (width 0.635) (layer F.Cu) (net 7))
 (via (at 155.956 29.464) (size 0.6858) (drill 0.3302) (layers F.Cu B.Cu) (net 15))
 (segment (start 168.576 38.1) (end 165.274 34.798) (width 0.635) (layer F.Cu) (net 15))
 (segment (start 159.512 34.798) (end 165.274 34.798) (width 0.635) (layer F.Cu) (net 15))
 (segment (start 155.956 31.242) (end 159.512 34.798) (width 0.635) (layer F.Cu) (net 15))
 (segment (start 155.956 31.242) (end 155.956 29.464) (width 0.635) (layer F.Cu) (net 15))
 (via (at 168.354 29.464) (size 0.6858) (drill 0.3302) (layers F.Cu B.Cu) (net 3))
 (segment (start 184.912 35.052) (end 181.864 35.052) (width 0.635) (layer F.Cu) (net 3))
 (segment (start 179.578 35.052) (end 181.864 35.052) (width 0.635) (layer F.Cu) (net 3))
 (segment (start 179.07 35.052) (end 179.578 35.052) (width 0.635) (layer F.Cu) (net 3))
 (segment (start 176.784 32.766) (end 179.07 35.052) (width 0.635) (layer F.Cu) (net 3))
 (segment (start 171.196 32.766) (end 176.784 32.766) (width 0.635) (layer F.Cu) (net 3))
 (segment (start 168.354 29.924) (end 171.196 32.766) (width 0.635) (layer F.Cu) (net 3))
 (segment (start 168.354 29.924) (end 168.354 29.464) (width 0.635) (layer F.Cu) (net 3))
 (segment (start 184.912 41.052) (end 185.516 41.052) (width 0.635) (layer F.Cu) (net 3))
 (segment (start 186.436 36.068) (end 185.42 35.052) (width 0.635) (layer F.Cu) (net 3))
 (segment (start 186.436 40.132) (end 186.436 36.068) (width 0.635) (layer F.Cu) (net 3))
 (segment (start 185.516 41.052) (end 186.436 40.132) (width 0.635) (layer F.Cu) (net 3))
 (segment (start 185.42 35.052) (end 184.912 35.052) (width 0.635) (layer F.Cu) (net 3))
 (via (at 185.42 51.562) (size 0.6858) (drill 0.3302) (layers F.Cu B.Cu) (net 13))
 (segment (start 198.912 37.052) (end 195.22 40.744) (width 0.635) (layer F.Cu) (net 13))
 (segment (start 195.22 48.68) (end 195.22 40.744) (width 0.635) (layer F.Cu) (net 13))
 (segment (start 194.89 49.01) (end 195.22 48.68) (width 0.635) (layer F.Cu) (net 13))
 (segment (start 187.718 49.01) (end 194.89 49.01) (width 0.635) (layer F.Cu) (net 13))
 (segment (start 187.718 49.01) (end 185.42 51.562) (width 0.635) (layer F.Cu) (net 13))
 (segment (start 198.912 37.052) (end 198.66 37.052) (width 0.635) (layer F.Cu) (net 13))
 (segment (start 213.868 28.448) (end 213.868 33.147) (width 0.635) (layer F.Cu) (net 13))
 (segment (start 213.868 33.147) (end 213.868 33.02) (width 0.635) (layer F.Cu) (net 13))
 (segment (start 213.868 33.02) (end 213.868 33.147) (width 0.635) (layer F.Cu) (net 13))
 (segment (start 198.912 37.052) (end 200.946 37.052) (width 0.635) (layer F.Cu) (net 13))
 (segment (start 202.311 33.147) (end 213.868 33.147) (width 0.635) (layer F.Cu) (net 13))
 (segment (start 201.93 33.528) (end 202.311 33.147) (width 0.635) (layer F.Cu) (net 13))
 (segment (start 201.93 36.068) (end 201.93 33.528) (width 0.635) (layer F.Cu) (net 13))
 (segment (start 200.946 37.052) (end 201.93 36.068) (width 0.635) (layer F.Cu) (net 13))
 (via (at 174.498 29.464) (size 0.6858) (drill 0.3302) (layers F.Cu B.Cu) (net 14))
 (segment (start 198.882 35.052) (end 197.612 33.782) (width 0.635) (layer F.Cu) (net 14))
 (segment (start 180.086 33.782) (end 197.612 33.782) (width 0.635) (layer F.Cu) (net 14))
 (segment (start 175.768 29.464) (end 180.086 33.782) (width 0.635) (layer F.Cu) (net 14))
 (segment (start 175.768 29.464) (end 174.498 29.464) (width 0.635) (layer F.Cu) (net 14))
 (segment (start 198.912 35.052) (end 200.279 35.052) (width 0.635) (layer F.Cu) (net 14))
 (segment (start 200.279 35.052) (end 201.142598 34.188402) (width 0.635) (layer F.Cu) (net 14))
 (segment (start 211.328 31.75) (end 211.328 28.448) (width 0.635) (layer F.Cu) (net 14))
 (segment (start 210.718402 32.359598) (end 211.328 31.75) (width 0.635) (layer F.Cu) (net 14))
 (segment (start 201.955402 32.359598) (end 210.718402 32.359598) (width 0.635) (layer F.Cu) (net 14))
 (segment (start 201.142598 33.172402) (end 201.955402 32.359598) (width 0.635) (layer F.Cu) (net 14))
 (segment (start 201.142598 34.188402) (end 201.142598 33.172402) (width 0.635) (layer F.Cu) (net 14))
 (segment (start 198.912 35.052) (end 199.771 35.052) (width 0.635) (layer F.Cu) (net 14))
 (segment (start 198.912 35.052) (end 199.898 35.052) (width 0.635) (layer F.Cu) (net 14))
 (segment (start 198.882 35.052) (end 198.912 35.052) (width 0.635) (layer F.Cu) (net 14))
 (via (at 191.096 51.566) (size 0.6858) (drill 0.3302) (layers F.Cu B.Cu) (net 12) (status 30))
 (segment (start 198.912 39.052) (end 196.02 41.944) (width 0.635) (layer F.Cu) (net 12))
 (segment (start 196.02 49.08) (end 196.02 41.944) (width 0.635) (layer F.Cu) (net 12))
 (segment (start 195.29 49.81) (end 196.02 49.08) (width 0.635) (layer F.Cu) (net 12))
 (segment (start 191.998 49.81) (end 195.29 49.81) (width 0.635) (layer F.Cu) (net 12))
 (segment (start 191.998 49.81) (end 191.262 51.308) (width 0.635) (layer F.Cu) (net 12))
 (via (at 207.264 50.292) (size 0.6858) (drill 0.3302) (layers F.Cu B.Cu) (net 11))
 (segment (start 198.912 41.052) (end 196.84 43.124) (width 0.635) (layer F.Cu) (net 11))
 (segment (start 196.84 50.23) (end 196.84 43.124) (width 0.635) (layer F.Cu) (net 11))
 (segment (start 197.74 51.13) (end 196.84 50.23) (width 0.635) (layer F.Cu) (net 11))
 (segment (start 206.426 51.13) (end 197.74 51.13) (width 0.635) (layer F.Cu) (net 11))
 (segment (start 206.426 51.13) (end 207.264 50.292) (width 0.635) (layer F.Cu) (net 11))
 (via (at 214.424 50.292) (size 0.6858) (drill 0.3302) (layers F.Cu B.Cu) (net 10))
 (segment (start 198.912 43.052) (end 198.308 43.052) (width 0.635) (layer F.Cu) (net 10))
 (segment (start 197.65 43.71) (end 198.308 43.052) (width 0.635) (layer F.Cu) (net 10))
 (segment (start 197.65 49.9) (end 197.65 43.71) (width 0.635) (layer F.Cu) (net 10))
 (segment (start 198.06 50.31) (end 197.65 49.9) (width 0.635) (layer F.Cu) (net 10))
 (segment (start 202.94 50.31) (end 198.06 50.31) (width 0.635) (layer F.Cu) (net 10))
 (segment (start 203.97 49.28) (end 202.94 50.31) (width 0.635) (layer F.Cu) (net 10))
 (segment (start 203.97 47.39) (end 203.97 49.28) (width 0.635) (layer F.Cu) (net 10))
 (segment (start 204.48 46.88) (end 203.97 47.39) (width 0.635) (layer F.Cu) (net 10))
 (segment (start 211.012 46.88) (end 204.48 46.88) (width 0.635) (layer F.Cu) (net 10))
 (segment (start 211.012 46.88) (end 214.424 50.292) (width 0.635) (layer F.Cu) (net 10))
 (segment (start 198.912 43.052) (end 201.55 43.052) (width 0.635) (layer F.Cu) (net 10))
 (segment (start 203.374 41.228) (end 203.374 34.544) (width 0.635) (layer F.Cu) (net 10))
 (segment (start 201.55 43.052) (end 203.374 41.228) (width 0.635) (layer F.Cu) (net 10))
 (segment (start 171.276 38.1) (end 181.61 38.1) (width 0.635) (layer F.Cu) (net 4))
 (segment (start 181.61 38.1) (end 182.658 37.052) (width 0.635) (layer F.Cu) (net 4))
 (segment (start 182.658 37.052) (end 184.912 37.052) (width 0.635) (layer F.Cu) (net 4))
 (segment (start 171.276 34.798) (end 171.276 38.1) (width 0.635) (layer F.Cu) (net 4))
 (segment (start 205.994 42.244) (end 203.628 42.244) (width 0.635) (layer F.Cu) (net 9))
 (segment (start 203.628 42.244) (end 200.82 45.052) (width 0.635) (layer F.Cu) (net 9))
 (segment (start 200.82 45.052) (end 198.912 45.052) (width 0.635) (layer F.Cu) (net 9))
 (segment (start 208.534 42.244) (end 208.534 42.926) (width 0.635) (layer F.Cu) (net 8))
 (segment (start 208.534 42.926) (end 207.772 43.688) (width 0.635) (layer F.Cu) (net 8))
 (segment (start 207.772 43.688) (end 203.962 43.688) (width 0.635) (layer F.Cu) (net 8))
 (segment (start 203.962 43.688) (end 200.598 47.052) (width 0.635) (layer F.Cu) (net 8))
 (segment (start 200.598 47.052) (end 198.912 47.052) (width 0.635) (layer F.Cu) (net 8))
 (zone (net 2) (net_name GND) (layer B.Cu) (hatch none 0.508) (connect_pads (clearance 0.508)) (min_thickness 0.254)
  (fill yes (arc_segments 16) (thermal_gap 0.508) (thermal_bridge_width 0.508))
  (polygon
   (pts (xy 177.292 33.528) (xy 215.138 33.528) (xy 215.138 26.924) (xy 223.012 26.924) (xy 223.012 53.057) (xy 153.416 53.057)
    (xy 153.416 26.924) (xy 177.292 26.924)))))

